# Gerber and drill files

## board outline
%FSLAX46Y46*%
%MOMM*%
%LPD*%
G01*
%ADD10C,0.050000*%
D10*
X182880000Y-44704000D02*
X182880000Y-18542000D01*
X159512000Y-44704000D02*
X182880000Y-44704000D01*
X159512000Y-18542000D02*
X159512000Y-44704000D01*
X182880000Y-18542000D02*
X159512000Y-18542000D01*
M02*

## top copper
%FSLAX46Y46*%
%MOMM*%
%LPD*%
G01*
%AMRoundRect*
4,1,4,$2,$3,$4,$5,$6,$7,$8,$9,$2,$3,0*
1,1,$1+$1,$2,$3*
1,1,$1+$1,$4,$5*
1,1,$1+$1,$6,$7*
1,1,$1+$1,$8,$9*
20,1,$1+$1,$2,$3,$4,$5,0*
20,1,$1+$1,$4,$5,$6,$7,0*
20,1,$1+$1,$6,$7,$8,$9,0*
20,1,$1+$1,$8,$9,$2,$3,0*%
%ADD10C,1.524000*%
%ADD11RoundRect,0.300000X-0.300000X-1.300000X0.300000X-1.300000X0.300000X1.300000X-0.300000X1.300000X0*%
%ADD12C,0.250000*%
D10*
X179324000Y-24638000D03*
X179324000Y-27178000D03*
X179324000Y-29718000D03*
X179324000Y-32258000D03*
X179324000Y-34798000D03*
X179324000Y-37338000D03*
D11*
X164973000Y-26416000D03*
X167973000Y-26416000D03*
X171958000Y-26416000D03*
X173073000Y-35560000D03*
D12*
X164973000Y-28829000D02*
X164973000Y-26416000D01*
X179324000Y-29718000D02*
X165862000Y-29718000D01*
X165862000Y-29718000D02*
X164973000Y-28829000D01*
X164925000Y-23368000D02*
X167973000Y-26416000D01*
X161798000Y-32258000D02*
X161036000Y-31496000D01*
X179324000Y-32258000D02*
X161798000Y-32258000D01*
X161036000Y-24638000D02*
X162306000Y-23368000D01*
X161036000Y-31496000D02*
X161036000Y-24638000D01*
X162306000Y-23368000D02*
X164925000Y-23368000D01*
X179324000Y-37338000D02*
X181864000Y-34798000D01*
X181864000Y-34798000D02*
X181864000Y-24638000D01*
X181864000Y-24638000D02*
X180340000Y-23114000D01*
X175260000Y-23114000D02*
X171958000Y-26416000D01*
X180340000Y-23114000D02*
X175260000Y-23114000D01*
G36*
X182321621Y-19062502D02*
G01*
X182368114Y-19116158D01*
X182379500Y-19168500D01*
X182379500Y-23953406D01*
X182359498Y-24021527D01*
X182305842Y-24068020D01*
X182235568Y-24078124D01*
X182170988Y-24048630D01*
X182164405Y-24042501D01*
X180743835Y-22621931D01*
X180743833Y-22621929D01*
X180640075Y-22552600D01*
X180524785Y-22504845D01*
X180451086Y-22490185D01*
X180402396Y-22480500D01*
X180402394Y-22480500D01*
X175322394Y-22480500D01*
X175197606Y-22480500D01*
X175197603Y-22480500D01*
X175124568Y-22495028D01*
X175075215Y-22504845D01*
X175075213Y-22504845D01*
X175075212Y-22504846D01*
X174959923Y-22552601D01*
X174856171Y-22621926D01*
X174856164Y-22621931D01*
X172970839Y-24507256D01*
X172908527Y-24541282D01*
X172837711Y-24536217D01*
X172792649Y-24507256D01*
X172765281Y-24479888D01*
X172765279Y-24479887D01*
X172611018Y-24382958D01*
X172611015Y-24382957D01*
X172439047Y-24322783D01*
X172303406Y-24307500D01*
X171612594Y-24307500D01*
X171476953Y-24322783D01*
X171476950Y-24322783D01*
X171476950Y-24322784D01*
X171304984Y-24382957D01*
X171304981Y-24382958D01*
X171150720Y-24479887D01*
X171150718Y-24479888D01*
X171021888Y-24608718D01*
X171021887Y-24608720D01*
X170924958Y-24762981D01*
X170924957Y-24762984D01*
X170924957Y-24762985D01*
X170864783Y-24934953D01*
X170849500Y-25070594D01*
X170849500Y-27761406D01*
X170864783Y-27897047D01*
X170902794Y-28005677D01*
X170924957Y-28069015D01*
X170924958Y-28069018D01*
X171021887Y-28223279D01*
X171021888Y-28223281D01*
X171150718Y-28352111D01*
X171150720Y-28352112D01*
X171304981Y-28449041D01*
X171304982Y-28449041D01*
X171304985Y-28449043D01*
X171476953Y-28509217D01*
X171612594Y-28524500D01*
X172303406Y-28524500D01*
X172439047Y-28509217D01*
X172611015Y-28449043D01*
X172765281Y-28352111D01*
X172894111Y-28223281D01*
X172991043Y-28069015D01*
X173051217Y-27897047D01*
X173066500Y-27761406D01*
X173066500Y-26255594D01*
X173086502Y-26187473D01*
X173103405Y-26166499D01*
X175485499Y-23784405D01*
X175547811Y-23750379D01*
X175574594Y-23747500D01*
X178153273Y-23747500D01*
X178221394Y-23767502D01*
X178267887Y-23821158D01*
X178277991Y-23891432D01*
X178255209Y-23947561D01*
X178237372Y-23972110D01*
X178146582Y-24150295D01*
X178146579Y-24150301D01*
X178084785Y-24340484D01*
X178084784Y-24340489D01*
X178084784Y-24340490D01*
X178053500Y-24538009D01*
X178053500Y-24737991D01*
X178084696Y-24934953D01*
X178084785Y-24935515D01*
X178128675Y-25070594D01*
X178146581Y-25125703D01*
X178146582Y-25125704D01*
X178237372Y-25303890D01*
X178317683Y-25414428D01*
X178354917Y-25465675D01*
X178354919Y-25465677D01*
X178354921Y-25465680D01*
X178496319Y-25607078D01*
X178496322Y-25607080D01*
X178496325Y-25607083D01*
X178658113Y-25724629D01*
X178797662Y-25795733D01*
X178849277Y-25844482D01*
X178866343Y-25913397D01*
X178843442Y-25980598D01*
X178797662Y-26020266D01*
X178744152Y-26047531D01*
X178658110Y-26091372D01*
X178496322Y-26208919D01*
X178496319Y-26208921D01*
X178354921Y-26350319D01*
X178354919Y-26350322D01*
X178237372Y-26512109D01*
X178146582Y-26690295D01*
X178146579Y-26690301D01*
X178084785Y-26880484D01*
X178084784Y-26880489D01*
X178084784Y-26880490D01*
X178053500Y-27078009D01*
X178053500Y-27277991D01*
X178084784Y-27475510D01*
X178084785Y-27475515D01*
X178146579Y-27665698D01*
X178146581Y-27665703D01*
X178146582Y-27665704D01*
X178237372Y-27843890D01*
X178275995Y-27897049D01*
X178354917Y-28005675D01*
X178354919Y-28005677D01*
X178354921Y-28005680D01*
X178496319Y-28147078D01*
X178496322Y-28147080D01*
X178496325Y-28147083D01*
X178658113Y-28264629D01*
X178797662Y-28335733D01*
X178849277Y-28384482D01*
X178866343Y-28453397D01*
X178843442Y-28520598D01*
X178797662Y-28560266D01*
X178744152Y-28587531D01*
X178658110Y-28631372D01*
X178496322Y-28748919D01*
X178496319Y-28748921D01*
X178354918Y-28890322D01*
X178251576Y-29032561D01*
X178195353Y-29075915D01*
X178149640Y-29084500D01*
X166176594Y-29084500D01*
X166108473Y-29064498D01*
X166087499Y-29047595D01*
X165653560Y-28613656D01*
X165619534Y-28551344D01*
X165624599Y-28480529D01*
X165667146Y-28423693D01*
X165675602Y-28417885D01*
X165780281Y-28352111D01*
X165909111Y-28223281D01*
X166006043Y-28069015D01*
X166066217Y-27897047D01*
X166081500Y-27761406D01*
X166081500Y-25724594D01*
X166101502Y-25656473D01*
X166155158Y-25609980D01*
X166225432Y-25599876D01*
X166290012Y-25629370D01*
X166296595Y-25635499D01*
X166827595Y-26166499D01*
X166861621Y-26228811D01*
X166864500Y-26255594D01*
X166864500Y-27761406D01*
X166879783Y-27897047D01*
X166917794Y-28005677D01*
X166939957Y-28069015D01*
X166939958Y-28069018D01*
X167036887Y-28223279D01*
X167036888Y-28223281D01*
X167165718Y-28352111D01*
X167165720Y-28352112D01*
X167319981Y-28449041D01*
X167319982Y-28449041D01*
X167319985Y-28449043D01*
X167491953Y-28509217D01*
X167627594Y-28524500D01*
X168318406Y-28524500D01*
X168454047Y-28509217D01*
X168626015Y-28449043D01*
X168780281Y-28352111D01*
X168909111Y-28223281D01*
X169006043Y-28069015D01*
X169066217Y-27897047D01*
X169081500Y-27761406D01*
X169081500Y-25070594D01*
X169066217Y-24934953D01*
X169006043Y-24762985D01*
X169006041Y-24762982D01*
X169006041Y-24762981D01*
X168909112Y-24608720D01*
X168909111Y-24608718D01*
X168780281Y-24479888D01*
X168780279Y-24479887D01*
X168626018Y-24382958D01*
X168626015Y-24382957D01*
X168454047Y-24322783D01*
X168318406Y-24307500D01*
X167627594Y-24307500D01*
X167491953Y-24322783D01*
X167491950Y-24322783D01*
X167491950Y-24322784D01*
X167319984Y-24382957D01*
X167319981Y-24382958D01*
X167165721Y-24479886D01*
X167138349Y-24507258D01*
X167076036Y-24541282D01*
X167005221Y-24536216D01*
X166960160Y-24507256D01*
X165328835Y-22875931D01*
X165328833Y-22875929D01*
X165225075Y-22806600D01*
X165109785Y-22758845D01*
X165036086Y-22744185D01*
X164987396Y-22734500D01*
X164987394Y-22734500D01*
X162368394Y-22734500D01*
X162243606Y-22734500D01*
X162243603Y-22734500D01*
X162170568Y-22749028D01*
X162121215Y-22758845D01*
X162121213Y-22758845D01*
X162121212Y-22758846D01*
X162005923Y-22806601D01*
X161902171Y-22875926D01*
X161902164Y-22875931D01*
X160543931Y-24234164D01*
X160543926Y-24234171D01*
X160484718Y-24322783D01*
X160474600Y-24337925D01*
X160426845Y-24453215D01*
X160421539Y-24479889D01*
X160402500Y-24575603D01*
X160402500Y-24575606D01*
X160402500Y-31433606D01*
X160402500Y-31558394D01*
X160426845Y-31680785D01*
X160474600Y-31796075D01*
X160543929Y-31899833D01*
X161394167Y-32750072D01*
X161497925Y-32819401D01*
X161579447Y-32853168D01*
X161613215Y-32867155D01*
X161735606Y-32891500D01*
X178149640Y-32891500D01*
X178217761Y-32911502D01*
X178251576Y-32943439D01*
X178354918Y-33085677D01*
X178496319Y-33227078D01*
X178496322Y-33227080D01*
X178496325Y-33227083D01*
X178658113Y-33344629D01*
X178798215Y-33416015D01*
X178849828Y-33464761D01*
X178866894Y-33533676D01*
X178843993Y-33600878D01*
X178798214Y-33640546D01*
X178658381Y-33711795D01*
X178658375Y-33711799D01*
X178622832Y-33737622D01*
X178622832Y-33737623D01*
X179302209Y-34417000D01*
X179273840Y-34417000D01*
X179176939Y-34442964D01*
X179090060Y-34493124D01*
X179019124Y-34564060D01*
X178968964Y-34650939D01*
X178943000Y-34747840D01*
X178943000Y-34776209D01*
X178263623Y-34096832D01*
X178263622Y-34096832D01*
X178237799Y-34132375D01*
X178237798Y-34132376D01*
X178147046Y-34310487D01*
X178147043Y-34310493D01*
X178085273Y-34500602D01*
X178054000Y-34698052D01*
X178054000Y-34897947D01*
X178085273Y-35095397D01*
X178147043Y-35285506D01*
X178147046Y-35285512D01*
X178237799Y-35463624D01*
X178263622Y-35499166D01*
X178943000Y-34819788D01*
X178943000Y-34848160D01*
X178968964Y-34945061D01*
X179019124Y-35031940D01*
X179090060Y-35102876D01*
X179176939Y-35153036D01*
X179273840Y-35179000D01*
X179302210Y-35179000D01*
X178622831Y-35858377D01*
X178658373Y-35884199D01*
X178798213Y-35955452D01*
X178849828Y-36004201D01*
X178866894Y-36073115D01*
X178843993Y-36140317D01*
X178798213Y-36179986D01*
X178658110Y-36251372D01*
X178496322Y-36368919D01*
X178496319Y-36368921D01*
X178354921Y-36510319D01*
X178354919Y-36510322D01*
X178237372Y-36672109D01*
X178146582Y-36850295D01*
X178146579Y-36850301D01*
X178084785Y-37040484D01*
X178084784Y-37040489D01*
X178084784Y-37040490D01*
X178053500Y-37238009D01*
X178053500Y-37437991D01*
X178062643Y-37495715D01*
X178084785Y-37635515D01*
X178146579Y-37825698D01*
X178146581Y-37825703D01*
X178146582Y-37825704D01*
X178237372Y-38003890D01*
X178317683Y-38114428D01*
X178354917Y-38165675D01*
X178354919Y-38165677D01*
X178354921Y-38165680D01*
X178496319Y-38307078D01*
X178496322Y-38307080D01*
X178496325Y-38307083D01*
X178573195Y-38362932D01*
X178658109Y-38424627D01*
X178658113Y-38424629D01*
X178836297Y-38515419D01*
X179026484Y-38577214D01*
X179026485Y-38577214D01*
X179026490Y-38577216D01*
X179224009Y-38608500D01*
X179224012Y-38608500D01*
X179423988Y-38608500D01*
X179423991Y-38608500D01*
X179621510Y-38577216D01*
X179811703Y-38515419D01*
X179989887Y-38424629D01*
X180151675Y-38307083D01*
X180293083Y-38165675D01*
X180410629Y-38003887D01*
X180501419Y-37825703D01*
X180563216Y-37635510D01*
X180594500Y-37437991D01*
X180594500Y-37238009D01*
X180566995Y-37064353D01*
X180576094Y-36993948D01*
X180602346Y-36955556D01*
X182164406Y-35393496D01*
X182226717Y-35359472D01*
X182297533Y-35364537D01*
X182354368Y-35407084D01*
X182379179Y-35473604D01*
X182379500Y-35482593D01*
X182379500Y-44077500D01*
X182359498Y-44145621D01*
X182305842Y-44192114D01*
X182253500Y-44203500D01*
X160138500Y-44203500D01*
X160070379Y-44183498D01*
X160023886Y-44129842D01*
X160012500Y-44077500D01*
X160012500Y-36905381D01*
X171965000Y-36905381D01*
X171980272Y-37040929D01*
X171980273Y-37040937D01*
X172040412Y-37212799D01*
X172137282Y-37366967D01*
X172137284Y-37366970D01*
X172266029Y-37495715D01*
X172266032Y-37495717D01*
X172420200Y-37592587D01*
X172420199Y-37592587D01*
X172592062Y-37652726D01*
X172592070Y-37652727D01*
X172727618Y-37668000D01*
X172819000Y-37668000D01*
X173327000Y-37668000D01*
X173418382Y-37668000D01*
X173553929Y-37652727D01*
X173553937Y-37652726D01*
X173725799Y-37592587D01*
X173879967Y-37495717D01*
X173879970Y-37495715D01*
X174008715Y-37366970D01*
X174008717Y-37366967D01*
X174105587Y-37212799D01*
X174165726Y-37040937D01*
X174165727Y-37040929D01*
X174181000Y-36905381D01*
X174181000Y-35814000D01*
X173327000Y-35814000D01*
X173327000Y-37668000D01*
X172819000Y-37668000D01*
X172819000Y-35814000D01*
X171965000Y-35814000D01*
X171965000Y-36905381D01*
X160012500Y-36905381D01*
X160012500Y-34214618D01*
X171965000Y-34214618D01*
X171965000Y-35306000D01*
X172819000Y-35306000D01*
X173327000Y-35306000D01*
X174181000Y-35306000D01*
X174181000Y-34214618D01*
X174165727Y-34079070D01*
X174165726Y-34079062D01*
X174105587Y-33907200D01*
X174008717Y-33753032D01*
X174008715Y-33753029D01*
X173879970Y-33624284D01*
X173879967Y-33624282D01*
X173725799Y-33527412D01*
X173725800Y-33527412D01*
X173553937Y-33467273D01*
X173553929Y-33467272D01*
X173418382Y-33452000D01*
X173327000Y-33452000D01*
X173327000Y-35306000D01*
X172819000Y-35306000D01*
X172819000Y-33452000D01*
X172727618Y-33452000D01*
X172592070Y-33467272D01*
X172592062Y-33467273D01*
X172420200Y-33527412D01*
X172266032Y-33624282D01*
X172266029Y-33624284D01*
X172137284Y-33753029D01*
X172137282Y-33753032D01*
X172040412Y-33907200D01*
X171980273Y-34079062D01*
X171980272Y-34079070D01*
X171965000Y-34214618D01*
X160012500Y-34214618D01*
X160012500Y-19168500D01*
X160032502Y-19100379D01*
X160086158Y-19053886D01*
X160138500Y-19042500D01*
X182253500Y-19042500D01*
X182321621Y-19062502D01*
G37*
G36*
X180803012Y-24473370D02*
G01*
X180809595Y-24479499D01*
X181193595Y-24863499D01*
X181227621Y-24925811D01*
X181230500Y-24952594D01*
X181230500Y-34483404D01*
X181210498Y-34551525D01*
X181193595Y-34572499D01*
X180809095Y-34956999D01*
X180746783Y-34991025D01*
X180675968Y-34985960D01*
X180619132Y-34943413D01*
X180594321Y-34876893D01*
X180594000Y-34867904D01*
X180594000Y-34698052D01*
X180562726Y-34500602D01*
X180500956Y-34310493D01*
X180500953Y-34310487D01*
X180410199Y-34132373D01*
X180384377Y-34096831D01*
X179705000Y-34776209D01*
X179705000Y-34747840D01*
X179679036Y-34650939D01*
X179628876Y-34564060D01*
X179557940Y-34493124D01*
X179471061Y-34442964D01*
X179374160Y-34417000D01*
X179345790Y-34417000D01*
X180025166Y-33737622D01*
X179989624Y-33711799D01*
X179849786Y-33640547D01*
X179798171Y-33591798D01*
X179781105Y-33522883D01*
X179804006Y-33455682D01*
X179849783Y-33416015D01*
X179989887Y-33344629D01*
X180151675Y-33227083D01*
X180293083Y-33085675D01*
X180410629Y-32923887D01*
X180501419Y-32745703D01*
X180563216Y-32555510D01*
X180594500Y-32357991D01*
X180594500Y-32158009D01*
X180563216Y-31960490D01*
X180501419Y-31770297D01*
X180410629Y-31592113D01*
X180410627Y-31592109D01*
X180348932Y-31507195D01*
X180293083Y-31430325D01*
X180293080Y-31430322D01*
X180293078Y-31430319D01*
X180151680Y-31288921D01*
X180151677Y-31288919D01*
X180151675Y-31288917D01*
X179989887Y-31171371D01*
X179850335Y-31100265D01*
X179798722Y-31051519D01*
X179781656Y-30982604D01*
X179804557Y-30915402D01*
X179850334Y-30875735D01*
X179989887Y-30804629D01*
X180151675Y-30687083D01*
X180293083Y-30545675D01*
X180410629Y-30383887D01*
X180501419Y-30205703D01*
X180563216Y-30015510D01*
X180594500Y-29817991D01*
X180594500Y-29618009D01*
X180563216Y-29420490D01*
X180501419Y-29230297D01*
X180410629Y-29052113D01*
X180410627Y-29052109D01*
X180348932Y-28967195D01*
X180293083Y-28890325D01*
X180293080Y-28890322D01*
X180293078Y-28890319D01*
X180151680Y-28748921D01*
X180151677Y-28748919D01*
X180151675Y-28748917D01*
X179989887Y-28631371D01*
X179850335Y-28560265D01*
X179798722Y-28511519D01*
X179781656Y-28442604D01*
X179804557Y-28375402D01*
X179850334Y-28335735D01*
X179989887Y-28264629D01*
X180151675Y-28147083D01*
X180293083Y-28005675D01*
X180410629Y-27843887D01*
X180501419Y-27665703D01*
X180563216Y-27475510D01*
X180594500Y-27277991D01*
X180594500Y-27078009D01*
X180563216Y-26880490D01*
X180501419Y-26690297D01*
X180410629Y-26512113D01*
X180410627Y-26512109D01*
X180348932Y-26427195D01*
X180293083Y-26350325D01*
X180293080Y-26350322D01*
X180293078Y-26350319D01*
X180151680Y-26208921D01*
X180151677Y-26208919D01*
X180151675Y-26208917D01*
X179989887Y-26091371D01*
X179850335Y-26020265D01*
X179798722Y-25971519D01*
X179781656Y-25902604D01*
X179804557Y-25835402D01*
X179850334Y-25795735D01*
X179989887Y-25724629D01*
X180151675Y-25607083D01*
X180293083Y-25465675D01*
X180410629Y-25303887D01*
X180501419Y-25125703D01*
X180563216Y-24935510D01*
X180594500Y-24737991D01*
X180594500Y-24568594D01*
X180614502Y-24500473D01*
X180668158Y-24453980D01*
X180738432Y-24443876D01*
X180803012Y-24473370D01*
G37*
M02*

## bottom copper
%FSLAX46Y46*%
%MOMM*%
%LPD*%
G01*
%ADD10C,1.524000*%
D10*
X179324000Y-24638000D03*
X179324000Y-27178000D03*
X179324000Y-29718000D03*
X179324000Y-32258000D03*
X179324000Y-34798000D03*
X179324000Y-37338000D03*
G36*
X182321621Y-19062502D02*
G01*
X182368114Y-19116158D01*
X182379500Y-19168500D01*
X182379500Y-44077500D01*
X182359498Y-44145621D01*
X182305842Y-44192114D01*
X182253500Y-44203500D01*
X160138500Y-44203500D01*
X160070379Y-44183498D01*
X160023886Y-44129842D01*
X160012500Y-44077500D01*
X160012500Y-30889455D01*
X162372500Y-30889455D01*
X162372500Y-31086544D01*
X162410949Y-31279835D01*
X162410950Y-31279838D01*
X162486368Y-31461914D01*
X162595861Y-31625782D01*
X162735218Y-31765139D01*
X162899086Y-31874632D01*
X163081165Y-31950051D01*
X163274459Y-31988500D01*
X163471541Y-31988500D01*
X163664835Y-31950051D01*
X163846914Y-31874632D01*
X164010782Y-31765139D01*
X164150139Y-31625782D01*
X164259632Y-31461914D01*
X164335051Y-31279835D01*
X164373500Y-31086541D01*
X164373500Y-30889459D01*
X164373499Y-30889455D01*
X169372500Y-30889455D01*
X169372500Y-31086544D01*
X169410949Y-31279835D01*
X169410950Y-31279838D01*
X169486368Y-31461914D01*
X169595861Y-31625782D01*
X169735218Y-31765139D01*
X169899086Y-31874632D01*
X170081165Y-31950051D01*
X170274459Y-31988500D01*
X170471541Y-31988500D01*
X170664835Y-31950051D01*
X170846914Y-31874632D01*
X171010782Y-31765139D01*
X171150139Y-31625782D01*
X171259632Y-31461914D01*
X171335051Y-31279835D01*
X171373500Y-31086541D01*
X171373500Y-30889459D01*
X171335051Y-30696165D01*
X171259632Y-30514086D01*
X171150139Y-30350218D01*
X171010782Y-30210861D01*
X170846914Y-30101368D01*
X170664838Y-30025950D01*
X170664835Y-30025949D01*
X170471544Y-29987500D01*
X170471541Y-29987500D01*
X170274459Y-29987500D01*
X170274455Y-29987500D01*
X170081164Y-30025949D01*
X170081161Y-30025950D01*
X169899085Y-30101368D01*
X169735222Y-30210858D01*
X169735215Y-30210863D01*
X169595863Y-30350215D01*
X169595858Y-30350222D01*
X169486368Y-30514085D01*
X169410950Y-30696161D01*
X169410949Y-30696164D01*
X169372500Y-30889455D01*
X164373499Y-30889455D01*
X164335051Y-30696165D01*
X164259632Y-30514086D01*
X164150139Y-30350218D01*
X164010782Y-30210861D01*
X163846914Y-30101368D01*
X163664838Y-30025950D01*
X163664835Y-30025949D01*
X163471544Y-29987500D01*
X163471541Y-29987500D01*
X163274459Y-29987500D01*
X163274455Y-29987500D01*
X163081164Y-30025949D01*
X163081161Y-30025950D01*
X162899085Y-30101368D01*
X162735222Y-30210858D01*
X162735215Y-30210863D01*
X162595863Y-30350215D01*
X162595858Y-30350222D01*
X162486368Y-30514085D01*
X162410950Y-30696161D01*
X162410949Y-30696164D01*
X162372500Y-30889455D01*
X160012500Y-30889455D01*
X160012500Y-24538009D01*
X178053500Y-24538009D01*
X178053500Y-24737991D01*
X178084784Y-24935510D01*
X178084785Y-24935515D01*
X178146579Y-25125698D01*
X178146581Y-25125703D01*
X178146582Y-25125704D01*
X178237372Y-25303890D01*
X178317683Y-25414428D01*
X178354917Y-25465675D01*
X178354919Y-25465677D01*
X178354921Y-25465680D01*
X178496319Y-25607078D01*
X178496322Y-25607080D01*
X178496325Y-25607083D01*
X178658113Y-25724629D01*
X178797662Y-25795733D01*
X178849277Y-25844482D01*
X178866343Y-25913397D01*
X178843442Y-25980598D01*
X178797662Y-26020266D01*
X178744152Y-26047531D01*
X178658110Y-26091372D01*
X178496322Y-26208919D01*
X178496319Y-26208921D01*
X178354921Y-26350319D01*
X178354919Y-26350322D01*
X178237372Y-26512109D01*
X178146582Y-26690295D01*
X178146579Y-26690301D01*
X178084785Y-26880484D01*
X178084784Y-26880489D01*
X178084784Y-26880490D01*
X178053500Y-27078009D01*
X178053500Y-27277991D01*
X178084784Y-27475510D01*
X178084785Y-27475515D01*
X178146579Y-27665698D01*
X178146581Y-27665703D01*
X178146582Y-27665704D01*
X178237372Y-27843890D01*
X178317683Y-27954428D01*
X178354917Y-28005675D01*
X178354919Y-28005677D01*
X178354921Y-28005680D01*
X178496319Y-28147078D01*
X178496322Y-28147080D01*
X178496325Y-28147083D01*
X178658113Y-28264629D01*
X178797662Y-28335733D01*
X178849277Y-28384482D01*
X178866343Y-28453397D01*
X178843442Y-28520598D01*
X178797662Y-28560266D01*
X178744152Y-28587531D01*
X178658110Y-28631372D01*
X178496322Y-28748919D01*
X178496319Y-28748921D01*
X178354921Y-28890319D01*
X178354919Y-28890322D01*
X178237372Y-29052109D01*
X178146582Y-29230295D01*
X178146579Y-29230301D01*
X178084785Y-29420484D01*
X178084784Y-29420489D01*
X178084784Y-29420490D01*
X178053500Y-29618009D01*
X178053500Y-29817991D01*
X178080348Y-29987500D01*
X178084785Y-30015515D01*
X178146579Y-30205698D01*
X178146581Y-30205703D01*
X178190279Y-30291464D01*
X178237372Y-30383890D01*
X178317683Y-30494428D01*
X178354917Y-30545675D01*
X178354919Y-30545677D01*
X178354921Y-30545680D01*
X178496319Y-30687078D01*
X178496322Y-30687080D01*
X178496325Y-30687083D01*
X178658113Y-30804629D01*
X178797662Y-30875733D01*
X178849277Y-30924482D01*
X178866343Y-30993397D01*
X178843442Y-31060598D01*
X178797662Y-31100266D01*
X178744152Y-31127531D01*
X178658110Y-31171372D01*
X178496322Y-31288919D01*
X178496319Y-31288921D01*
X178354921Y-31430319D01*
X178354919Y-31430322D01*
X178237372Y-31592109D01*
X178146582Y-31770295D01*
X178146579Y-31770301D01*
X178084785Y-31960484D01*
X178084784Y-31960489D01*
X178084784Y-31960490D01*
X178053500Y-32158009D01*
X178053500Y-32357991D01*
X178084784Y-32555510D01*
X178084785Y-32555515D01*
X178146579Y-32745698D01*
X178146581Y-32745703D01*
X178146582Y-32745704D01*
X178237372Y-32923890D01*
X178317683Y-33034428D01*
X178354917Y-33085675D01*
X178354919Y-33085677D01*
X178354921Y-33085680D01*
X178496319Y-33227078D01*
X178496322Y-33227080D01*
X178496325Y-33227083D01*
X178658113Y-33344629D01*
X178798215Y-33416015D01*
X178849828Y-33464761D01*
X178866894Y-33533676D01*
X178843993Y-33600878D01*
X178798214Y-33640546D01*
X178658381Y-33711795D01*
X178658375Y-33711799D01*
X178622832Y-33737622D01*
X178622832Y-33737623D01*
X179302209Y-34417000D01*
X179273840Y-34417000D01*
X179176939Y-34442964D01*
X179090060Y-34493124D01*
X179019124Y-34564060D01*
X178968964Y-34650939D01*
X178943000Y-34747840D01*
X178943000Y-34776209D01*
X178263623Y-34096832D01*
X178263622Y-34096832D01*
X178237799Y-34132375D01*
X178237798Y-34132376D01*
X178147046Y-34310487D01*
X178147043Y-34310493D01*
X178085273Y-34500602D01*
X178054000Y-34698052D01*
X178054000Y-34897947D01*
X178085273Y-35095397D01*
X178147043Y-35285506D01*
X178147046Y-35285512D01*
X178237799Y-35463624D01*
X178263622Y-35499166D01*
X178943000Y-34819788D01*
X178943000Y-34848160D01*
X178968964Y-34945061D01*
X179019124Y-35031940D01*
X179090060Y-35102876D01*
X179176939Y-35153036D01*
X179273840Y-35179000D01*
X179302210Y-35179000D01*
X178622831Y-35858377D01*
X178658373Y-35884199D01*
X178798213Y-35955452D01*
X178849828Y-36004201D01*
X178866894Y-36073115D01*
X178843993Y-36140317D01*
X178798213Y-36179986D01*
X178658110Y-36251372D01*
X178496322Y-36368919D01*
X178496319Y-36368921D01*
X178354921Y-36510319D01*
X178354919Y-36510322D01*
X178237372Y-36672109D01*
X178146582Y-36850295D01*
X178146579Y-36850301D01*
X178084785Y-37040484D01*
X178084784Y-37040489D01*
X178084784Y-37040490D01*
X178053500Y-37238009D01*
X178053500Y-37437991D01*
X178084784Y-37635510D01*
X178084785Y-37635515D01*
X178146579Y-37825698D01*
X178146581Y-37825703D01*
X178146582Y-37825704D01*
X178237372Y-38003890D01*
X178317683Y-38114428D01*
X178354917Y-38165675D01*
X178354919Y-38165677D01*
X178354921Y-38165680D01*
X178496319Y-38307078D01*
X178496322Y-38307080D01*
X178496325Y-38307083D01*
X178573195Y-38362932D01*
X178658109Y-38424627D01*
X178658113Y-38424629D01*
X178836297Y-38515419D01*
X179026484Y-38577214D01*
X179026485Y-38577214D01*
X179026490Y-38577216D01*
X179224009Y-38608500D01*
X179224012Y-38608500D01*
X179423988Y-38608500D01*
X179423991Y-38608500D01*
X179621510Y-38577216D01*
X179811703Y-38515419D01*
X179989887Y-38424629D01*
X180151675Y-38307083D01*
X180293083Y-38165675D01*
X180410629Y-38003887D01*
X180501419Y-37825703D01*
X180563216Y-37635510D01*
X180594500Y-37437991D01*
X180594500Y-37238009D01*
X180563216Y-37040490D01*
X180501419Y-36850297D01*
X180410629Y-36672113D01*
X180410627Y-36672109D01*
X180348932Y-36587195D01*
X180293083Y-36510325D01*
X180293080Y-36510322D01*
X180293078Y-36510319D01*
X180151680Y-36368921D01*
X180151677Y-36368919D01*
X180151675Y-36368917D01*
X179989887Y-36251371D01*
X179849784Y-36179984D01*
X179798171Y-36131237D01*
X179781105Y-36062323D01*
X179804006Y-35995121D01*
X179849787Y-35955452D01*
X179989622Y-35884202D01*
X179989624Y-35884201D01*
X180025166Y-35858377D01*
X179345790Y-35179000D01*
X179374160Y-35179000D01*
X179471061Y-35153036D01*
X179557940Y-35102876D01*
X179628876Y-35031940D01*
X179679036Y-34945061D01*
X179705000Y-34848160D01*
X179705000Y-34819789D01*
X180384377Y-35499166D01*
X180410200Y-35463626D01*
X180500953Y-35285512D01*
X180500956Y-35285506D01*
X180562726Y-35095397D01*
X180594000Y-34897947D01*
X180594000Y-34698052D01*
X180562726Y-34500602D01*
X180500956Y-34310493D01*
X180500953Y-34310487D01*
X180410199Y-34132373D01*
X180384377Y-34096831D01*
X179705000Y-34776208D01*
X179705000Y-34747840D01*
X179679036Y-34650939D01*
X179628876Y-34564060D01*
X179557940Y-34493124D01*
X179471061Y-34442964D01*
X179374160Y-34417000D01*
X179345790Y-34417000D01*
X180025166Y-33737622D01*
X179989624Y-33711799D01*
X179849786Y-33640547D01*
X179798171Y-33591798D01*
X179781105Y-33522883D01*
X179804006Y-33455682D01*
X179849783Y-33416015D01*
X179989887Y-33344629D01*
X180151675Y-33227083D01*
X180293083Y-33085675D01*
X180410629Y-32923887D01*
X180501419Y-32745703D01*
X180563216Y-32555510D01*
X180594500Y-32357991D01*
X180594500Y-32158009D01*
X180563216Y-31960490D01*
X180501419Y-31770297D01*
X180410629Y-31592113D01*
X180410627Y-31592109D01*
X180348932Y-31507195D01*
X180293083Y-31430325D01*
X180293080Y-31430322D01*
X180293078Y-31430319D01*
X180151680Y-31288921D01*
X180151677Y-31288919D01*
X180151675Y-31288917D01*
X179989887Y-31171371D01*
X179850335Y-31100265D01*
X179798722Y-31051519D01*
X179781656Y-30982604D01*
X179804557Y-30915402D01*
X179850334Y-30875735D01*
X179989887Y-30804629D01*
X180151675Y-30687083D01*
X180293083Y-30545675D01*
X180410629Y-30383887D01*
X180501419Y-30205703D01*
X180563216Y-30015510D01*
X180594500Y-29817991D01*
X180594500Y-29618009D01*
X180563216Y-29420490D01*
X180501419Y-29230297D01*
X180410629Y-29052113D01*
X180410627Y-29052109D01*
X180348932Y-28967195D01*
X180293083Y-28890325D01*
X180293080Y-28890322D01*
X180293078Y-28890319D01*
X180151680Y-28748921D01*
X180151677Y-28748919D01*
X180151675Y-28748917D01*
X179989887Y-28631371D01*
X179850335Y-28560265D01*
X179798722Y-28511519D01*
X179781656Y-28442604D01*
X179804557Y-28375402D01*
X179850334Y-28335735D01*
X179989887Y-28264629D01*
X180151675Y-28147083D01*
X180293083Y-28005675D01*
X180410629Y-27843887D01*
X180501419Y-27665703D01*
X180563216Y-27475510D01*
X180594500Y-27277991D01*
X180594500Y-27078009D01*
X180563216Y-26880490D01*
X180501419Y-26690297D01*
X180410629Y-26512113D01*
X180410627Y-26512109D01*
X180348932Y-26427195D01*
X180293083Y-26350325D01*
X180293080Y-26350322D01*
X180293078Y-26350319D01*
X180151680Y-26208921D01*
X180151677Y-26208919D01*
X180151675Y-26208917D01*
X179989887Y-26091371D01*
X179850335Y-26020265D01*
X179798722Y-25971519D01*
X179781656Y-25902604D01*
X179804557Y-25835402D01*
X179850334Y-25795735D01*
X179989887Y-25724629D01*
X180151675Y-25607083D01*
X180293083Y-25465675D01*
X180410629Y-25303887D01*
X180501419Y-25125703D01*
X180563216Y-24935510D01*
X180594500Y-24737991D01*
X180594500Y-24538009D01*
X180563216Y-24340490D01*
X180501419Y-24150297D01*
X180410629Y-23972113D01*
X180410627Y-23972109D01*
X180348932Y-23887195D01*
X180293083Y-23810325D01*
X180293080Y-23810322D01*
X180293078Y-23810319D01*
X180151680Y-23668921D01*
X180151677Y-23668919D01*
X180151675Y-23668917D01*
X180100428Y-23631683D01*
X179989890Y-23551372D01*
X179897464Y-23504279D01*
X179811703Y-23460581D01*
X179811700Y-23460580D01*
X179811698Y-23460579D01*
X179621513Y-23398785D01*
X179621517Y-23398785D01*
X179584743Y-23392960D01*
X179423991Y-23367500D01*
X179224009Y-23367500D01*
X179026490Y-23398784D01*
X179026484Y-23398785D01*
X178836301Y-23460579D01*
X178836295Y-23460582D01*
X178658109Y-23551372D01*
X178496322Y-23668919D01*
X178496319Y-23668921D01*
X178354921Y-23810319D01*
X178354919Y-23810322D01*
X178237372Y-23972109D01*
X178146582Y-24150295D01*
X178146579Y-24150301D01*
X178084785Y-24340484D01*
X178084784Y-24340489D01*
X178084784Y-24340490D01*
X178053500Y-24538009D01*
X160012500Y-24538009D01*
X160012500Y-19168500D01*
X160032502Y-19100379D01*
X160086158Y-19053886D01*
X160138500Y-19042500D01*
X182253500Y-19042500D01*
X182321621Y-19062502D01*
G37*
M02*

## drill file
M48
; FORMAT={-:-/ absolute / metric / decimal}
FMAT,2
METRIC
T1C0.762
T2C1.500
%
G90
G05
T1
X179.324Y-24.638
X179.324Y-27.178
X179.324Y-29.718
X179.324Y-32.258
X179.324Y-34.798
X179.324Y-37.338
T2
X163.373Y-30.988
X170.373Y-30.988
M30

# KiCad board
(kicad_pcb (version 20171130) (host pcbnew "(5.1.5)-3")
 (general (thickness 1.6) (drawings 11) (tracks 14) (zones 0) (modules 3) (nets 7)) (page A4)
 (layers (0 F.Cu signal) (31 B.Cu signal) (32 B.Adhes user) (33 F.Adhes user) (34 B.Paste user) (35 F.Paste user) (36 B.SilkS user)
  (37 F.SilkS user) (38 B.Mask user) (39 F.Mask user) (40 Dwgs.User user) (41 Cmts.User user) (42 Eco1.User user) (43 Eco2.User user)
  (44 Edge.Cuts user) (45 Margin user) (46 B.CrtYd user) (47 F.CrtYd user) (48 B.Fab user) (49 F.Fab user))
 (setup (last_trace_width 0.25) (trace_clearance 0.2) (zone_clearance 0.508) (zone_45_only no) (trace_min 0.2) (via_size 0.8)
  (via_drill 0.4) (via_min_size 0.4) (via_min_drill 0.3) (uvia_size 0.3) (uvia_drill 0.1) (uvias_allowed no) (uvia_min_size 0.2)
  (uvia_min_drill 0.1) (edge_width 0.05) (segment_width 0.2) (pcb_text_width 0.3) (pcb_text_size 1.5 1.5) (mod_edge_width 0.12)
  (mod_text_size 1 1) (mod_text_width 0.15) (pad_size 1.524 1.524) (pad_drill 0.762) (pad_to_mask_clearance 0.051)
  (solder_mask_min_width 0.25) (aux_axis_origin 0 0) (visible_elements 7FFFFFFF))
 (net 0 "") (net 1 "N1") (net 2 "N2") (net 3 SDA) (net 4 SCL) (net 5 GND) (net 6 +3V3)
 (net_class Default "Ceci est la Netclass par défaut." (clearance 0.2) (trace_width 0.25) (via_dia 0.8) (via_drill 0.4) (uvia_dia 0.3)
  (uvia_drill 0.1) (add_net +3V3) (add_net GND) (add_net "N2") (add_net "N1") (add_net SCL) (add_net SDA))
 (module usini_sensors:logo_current (layer B.Cu) (at 175.768 23.241 180)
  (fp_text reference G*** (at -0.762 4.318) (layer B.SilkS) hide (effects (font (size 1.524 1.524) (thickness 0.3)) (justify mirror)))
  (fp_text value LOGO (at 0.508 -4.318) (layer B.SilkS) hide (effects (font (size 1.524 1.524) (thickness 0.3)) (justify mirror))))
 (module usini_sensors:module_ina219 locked (layer F.Cu) (at 179.324 24.638 180)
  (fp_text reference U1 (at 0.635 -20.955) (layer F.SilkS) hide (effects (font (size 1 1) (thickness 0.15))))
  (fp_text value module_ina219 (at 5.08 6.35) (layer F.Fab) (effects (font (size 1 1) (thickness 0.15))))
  (pad 6 thru_hole circle (at 0 0 180) (size 1.524 1.524) (drill 0.762) (layers *.Cu *.Mask) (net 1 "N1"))
  (pad 5 thru_hole circle (at 0 -2.54 180) (size 1.524 1.524) (drill 0.762) (layers *.Cu *.Mask) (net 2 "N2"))
  (pad 4 thru_hole circle (at 0 -5.08 180) (size 1.524 1.524) (drill 0.762) (layers *.Cu *.Mask) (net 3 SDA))
  (pad 3 thru_hole circle (at 0 -7.62 180) (size 1.524 1.524) (drill 0.762) (layers *.Cu *.Mask) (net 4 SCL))
  (pad 2 thru_hole circle (at 0 -10.16 180) (size 1.524 1.524) (drill 0.762) (layers *.Cu *.Mask) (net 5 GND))
  (pad 1 thru_hole circle (at 0 -12.7 180) (size 1.524 1.524) (drill 0.762) (layers *.Cu *.Mask) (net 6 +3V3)))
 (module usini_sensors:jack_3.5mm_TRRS (layer F.Cu) (at 168.148 30.988)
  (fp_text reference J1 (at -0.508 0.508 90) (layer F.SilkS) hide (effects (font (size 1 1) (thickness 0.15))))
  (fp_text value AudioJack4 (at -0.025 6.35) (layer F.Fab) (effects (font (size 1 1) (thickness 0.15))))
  (pad "" np_thru_hole circle (at 2.225 0) (size 1.5 1.5) (drill 1.5) (layers *.Cu *.Mask))
  (pad "" np_thru_hole circle (at -4.775 0) (size 1.5 1.5) (drill 1.5) (layers *.Cu *.Mask))
  (pad R2 smd roundrect (at -3.175 -4.572) (size 1.2 3.2) (layers F.Cu F.Paste F.Mask) (roundrect_rratio 0.25) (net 3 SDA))
  (pad R1 smd roundrect (at -0.175 -4.572) (size 1.2 3.2) (layers F.Cu F.Paste F.Mask) (roundrect_rratio 0.25) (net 4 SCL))
  (pad T smd roundrect (at 3.81 -4.572) (size 1.2 3.2) (layers F.Cu F.Paste F.Mask) (roundrect_rratio 0.25) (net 6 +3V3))
  (pad S smd roundrect (at 4.925 4.572) (size 1.2 3.2) (layers F.Cu F.Paste F.Mask) (roundrect_rratio 0.25) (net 5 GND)))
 (gr_line (start 182.88 44.704) (end 182.88 18.542) (layer Edge.Cuts) (width 0.05))
 (gr_line (start 159.512 44.704) (end 182.88 44.704) (layer Edge.Cuts) (width 0.05))
 (gr_line (start 159.512 18.542) (end 159.512 44.704) (layer Edge.Cuts) (width 0.05))
 (gr_line (start 182.88 18.542) (end 159.512 18.542) (layer Edge.Cuts) (width 0.05))
 (segment (start 164.973 28.829) (end 164.973 26.416) (width 0.25) (layer F.Cu) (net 3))
 (segment (start 179.324 29.718) (end 165.862 29.718) (width 0.25) (layer F.Cu) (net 3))
 (segment (start 165.862 29.718) (end 164.973 28.829) (width 0.25) (layer F.Cu) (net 3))
 (segment (start 164.925 23.368) (end 167.973 26.416) (width 0.25) (layer F.Cu) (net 4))
 (segment (start 161.798 32.258) (end 161.036 31.496) (width 0.25) (layer F.Cu) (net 4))
 (segment (start 179.324 32.258) (end 161.798 32.258) (width 0.25) (layer F.Cu) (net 4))
 (segment (start 161.036 24.638) (end 162.306 23.368) (width 0.25) (layer F.Cu) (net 4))
 (segment (start 161.036 31.496) (end 161.036 24.638) (width 0.25) (layer F.Cu) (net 4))
 (segment (start 162.306 23.368) (end 164.925 23.368) (width 0.25) (layer F.Cu) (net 4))
 (segment (start 179.324 37.338) (end 181.864 34.798) (width 0.25) (layer F.Cu) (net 6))
 (segment (start 181.864 34.798) (end 181.864 24.638) (width 0.25) (layer F.Cu) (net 6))
 (segment (start 181.864 24.638) (end 180.34 23.114) (width 0.25) (layer F.Cu) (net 6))
 (segment (start 175.26 23.114) (end 171.958 26.416) (width 0.25) (layer F.Cu) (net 6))
 (segment (start 180.34 23.114) (end 175.26 23.114) (width 0.25) (layer F.Cu) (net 6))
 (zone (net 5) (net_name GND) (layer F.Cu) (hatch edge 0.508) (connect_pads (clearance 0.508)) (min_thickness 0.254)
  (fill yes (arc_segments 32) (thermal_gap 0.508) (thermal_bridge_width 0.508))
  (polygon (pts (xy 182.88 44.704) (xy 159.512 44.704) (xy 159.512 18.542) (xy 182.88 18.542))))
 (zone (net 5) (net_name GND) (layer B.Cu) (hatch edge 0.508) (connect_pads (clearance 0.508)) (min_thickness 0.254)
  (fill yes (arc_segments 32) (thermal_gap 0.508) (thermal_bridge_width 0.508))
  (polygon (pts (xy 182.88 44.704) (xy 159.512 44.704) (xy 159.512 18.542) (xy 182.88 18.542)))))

